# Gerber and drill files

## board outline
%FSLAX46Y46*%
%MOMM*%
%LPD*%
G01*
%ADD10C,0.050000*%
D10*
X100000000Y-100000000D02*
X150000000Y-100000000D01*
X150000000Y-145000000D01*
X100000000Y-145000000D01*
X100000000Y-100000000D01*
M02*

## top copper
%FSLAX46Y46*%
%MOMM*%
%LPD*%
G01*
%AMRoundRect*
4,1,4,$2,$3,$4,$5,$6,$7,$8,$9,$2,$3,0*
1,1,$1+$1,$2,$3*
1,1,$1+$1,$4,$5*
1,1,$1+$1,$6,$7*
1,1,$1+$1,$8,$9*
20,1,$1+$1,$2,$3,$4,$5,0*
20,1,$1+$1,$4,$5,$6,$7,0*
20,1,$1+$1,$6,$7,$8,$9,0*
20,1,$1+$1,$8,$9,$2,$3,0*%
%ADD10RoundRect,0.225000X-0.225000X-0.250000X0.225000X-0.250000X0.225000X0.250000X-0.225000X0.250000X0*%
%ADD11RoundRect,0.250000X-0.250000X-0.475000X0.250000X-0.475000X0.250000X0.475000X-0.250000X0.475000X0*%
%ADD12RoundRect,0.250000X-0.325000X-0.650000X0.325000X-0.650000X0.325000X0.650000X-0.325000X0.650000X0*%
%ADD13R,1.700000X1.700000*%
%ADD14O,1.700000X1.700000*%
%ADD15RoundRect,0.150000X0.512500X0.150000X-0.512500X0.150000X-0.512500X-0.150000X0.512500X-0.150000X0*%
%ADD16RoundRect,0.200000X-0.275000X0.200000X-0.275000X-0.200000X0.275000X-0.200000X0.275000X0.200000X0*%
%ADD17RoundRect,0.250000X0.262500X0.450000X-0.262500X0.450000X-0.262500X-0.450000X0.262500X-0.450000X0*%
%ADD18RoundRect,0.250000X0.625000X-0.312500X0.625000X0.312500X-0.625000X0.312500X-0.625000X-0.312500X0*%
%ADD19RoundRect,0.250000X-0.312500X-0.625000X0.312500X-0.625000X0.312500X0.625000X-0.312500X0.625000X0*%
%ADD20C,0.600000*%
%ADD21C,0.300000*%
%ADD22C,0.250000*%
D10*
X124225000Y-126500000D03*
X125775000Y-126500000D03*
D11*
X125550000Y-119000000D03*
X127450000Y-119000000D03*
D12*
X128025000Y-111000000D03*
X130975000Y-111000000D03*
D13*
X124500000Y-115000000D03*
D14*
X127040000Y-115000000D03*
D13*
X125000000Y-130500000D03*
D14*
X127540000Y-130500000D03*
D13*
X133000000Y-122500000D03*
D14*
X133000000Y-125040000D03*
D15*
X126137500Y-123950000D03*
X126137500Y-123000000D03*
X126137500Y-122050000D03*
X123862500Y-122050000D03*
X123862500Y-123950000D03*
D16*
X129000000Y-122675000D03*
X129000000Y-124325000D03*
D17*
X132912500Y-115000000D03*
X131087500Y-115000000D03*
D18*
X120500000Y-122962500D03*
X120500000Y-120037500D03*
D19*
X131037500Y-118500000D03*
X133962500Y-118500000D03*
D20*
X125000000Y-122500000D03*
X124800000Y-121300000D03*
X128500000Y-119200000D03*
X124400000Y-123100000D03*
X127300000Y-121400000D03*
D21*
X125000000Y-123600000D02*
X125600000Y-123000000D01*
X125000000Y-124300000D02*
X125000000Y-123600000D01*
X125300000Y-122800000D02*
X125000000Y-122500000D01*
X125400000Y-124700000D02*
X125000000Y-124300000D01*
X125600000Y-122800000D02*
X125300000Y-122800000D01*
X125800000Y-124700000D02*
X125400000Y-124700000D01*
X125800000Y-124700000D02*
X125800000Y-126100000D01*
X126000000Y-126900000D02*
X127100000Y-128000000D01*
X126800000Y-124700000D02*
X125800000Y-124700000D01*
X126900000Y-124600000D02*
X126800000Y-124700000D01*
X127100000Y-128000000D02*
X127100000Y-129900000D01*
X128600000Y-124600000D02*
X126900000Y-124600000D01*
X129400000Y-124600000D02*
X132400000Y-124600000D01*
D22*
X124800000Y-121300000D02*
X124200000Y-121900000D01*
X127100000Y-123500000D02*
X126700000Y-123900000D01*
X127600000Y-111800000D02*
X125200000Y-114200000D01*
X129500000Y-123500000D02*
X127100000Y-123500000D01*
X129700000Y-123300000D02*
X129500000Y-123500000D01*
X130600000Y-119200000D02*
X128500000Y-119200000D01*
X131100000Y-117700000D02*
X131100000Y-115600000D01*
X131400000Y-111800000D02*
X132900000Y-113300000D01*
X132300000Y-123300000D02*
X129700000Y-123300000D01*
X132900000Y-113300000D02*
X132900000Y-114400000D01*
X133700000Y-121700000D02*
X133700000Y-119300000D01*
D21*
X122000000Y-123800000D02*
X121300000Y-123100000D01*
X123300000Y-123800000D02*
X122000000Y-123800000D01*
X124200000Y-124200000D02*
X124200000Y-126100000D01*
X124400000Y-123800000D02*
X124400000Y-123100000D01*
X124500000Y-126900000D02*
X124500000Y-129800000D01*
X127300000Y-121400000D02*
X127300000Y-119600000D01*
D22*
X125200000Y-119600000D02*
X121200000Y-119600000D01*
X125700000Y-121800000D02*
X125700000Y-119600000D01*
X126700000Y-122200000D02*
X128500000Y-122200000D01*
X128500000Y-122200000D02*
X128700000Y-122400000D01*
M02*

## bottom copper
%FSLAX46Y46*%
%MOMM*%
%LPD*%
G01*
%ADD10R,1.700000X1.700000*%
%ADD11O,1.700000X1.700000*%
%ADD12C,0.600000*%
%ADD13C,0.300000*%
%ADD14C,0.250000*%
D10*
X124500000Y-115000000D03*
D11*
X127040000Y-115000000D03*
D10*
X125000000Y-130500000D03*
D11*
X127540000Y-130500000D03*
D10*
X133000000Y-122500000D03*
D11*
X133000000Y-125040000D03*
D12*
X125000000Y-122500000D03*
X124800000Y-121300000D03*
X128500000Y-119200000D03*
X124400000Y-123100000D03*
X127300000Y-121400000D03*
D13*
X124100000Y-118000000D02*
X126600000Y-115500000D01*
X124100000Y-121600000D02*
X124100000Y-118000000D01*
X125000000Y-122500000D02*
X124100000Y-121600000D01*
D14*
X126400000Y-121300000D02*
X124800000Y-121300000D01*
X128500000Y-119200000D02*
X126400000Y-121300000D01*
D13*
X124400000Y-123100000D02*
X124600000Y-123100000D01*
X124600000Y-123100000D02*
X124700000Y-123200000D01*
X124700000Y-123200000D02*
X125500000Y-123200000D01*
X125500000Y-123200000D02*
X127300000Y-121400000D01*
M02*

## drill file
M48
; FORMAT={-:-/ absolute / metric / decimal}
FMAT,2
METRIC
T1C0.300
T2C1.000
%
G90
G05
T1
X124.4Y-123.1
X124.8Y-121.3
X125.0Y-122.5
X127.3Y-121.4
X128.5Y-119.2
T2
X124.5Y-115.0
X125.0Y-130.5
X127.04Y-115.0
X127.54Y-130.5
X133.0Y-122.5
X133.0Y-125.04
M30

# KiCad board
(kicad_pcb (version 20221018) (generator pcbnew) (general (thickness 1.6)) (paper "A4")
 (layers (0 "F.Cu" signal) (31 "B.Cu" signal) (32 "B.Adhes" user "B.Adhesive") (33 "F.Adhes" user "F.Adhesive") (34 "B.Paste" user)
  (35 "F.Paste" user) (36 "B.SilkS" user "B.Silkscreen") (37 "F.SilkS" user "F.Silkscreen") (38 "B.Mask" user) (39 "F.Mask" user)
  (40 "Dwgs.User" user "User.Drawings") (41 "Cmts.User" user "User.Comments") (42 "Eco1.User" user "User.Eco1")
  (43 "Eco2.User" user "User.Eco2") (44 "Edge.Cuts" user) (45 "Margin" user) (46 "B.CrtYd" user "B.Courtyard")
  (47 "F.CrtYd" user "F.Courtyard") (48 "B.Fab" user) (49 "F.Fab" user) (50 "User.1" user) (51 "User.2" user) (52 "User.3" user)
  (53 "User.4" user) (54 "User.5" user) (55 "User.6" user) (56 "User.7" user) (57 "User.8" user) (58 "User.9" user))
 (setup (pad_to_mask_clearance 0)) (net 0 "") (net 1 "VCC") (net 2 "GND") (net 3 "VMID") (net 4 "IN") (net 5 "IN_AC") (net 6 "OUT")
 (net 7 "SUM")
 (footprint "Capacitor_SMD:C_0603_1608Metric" (layer "F.Cu") (at 125 126.5)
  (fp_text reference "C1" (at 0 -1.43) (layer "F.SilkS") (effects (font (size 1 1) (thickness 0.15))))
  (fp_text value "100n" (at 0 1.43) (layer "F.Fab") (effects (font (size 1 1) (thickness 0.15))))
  (pad "1" smd roundrect (at -0.775 0) (size 0.9 0.95) (layers "F.Cu" "F.Paste" "F.Mask") (roundrect_rratio 0.25) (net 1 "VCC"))
  (pad "2" smd roundrect (at 0.775 0) (size 0.9 0.95) (layers "F.Cu" "F.Paste" "F.Mask") (roundrect_rratio 0.25) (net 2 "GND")))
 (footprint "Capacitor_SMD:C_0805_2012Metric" (layer "F.Cu") (at 126.5 119)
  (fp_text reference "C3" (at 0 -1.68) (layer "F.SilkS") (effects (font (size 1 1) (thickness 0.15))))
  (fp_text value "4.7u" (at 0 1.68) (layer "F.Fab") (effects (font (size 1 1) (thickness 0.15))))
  (pad "1" smd roundrect (at -0.95 0) (size 1 1.45) (layers "F.Cu" "F.Paste" "F.Mask") (roundrect_rratio 0.25) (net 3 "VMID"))
  (pad "2" smd roundrect (at 0.95 0) (size 1 1.45) (layers "F.Cu" "F.Paste" "F.Mask") (roundrect_rratio 0.25) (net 1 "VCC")))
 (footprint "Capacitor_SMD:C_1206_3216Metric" (layer "F.Cu") (at 129.5 111)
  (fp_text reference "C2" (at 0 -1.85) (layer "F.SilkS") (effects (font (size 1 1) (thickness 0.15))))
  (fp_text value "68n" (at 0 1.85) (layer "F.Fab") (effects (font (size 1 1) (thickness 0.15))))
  (pad "1" smd roundrect (at -1.475 0) (size 1.15 1.8) (layers "F.Cu" "F.Paste" "F.Mask") (roundrect_rratio 0.217391) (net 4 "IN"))
  (pad "2" smd roundrect (at 1.475 0) (size 1.15 1.8) (layers "F.Cu" "F.Paste" "F.Mask") (roundrect_rratio 0.217391) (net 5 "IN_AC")))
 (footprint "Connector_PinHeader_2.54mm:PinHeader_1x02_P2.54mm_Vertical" (layer "F.Cu") (at 124.5 115 90)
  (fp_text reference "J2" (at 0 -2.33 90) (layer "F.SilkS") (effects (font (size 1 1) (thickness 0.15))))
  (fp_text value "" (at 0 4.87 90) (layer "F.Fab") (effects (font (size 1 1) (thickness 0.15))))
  (pad "1" thru_hole rect (at 0 0 90) (size 1.7 1.7) (drill 1) (layers "*.Cu" "*.Mask") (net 4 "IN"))
  (pad "2" thru_hole oval (at 0 2.54 90) (size 1.7 1.7) (drill 1) (layers "*.Cu" "*.Mask") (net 2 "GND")))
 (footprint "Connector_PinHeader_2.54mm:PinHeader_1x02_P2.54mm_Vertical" (layer "F.Cu") (at 125 130.5 90)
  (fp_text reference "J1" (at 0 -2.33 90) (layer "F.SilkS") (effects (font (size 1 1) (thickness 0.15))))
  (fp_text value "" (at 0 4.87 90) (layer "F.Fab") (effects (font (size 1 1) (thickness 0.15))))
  (pad "1" thru_hole rect (at 0 0 90) (size 1.7 1.7) (drill 1) (layers "*.Cu" "*.Mask") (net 1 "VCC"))
  (pad "2" thru_hole oval (at 0 2.54 90) (size 1.7 1.7) (drill 1) (layers "*.Cu" "*.Mask") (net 2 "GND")))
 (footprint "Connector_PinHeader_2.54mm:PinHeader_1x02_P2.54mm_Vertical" (layer "F.Cu") (at 133 122.5)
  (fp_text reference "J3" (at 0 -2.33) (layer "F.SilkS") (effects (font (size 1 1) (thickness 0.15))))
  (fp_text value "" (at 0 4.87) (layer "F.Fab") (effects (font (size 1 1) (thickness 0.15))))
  (pad "1" thru_hole rect (at 0 0) (size 1.7 1.7) (drill 1) (layers "*.Cu" "*.Mask") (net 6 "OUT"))
  (pad "2" thru_hole oval (at 0 2.54) (size 1.7 1.7) (drill 1) (layers "*.Cu" "*.Mask") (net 2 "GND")))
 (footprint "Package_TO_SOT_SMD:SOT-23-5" (layer "F.Cu") (at 125 123 180)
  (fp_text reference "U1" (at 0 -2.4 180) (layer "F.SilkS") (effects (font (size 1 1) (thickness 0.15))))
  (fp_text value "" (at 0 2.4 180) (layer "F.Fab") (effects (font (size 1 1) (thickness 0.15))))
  (pad "1" smd roundrect (at -1.1375 -0.95 180) (size 1.325 0.6) (layers "F.Cu" "F.Paste" "F.Mask") (roundrect_rratio 0.25) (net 6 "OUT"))
  (pad "2" smd roundrect (at -1.1375 0 180) (size 1.325 0.6) (layers "F.Cu" "F.Paste" "F.Mask") (roundrect_rratio 0.25) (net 2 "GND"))
  (pad "3" smd roundrect (at -1.1375 0.95 180) (size 1.325 0.6) (layers "F.Cu" "F.Paste" "F.Mask") (roundrect_rratio 0.25) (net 3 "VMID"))
  (pad "4" smd roundrect (at 1.1375 0.95 180) (size 1.325 0.6) (layers "F.Cu" "F.Paste" "F.Mask") (roundrect_rratio 0.25) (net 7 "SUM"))
  (pad "5" smd roundrect (at 1.1375 -0.95 180) (size 1.325 0.6) (layers "F.Cu" "F.Paste" "F.Mask") (roundrect_rratio 0.25) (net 1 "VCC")))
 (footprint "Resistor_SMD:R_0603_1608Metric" (layer "F.Cu") (at 129 123.5 -90)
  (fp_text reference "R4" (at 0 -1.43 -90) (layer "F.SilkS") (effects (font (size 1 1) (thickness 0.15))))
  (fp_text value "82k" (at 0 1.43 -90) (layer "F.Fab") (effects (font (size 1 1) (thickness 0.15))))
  (pad "1" smd roundrect (at -0.825 0 270) (size 0.8 0.95) (layers "F.Cu" "F.Paste" "F.Mask") (roundrect_rratio 0.25) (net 3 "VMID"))
  (pad "2" smd roundrect (at 0.825 0 270) (size 0.8 0.95) (layers "F.Cu" "F.Paste" "F.Mask") (roundrect_rratio 0.25) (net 2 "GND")))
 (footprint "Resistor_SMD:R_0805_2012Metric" (layer "F.Cu") (at 132 115 180)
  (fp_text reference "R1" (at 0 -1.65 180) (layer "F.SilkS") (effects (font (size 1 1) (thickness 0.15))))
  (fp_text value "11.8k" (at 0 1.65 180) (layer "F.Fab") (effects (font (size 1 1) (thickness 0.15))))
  (pad "1" smd roundrect (at -0.9125 0 180) (size 1.025 1.4) (layers "F.Cu" "F.Paste" "F.Mask") (roundrect_rratio 0.243902) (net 5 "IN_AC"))
  (pad "2" smd roundrect (at 0.9125 0 180) (size 1.025 1.4) (layers "F.Cu" "F.Paste" "F.Mask") (roundrect_rratio 0.243902) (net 7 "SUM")))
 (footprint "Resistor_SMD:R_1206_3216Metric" (layer "F.Cu") (at 120.5 121.5 90)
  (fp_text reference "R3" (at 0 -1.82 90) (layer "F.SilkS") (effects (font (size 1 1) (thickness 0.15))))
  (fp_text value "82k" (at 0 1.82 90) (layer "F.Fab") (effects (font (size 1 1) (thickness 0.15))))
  (pad "1" smd roundrect (at -1.4625 0 90) (size 1.125 1.75) (layers "F.Cu" "F.Paste" "F.Mask") (roundrect_rratio 0.222222) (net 1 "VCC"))
  (pad "2" smd roundrect (at 1.4625 0 90) (size 1.125 1.75) (layers "F.Cu" "F.Paste" "F.Mask") (roundrect_rratio 0.222222) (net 3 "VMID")))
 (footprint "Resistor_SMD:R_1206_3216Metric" (layer "F.Cu") (at 132.5 118.5)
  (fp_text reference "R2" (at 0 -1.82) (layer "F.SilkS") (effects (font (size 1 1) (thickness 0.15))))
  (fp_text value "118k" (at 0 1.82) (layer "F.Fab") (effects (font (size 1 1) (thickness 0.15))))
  (pad "1" smd roundrect (at -1.4625 0) (size 1.125 1.75) (layers "F.Cu" "F.Paste" "F.Mask") (roundrect_rratio 0.222222) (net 7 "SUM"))
  (pad "2" smd roundrect (at 1.4625 0) (size 1.125 1.75) (layers "F.Cu" "F.Paste" "F.Mask") (roundrect_rratio 0.222222) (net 6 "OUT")))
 (gr_rect (start 100 100) (end 150 145) (stroke (width 0.05) (type default)) (fill none) (layer "Edge.Cuts"))
 (segment (start 125 123.6) (end 125.6 123) (width 0.3) (layer "F.Cu") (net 2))
 (segment (start 125 124.3) (end 125 123.6) (width 0.3) (layer "F.Cu") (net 2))
 (segment (start 125.3 122.8) (end 125 122.5) (width 0.3) (layer "F.Cu") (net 2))
 (segment (start 125.4 124.7) (end 125 124.3) (width 0.3) (layer "F.Cu") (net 2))
 (segment (start 125.6 122.8) (end 125.3 122.8) (width 0.3) (layer "F.Cu") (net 2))
 (segment (start 125.8 124.7) (end 125.4 124.7) (width 0.3) (layer "F.Cu") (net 2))
 (segment (start 125.8 124.7) (end 125.8 126.1) (width 0.3) (layer "F.Cu") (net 2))
 (segment (start 126 126.9) (end 127.1 128) (width 0.3) (layer "F.Cu") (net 2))
 (segment (start 126.8 124.7) (end 125.8 124.7) (width 0.3) (layer "F.Cu") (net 2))
 (segment (start 126.9 124.6) (end 126.8 124.7) (width 0.3) (layer "F.Cu") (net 2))
 (segment (start 127.1 128) (end 127.1 129.9) (width 0.3) (layer "F.Cu") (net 2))
 (segment (start 128.6 124.6) (end 126.9 124.6) (width 0.3) (layer "F.Cu") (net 2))
 (segment (start 129.4 124.6) (end 132.4 124.6) (width 0.3) (layer "F.Cu") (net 2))
 (via (at 125 122.5) (size 0.6) (drill 0.3) (layers "F.Cu" "B.Cu") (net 2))
 (segment (start 124.1 118) (end 126.6 115.5) (width 0.3) (layer "B.Cu") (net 2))
 (segment (start 124.1 121.6) (end 124.1 118) (width 0.3) (layer "B.Cu") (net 2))
 (segment (start 124.8 121.3) (end 124.2 121.9) (width 0.25) (layer "F.Cu") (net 7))
 (segment (start 125 122.5) (end 124.1 121.6) (width 0.3) (layer "B.Cu") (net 2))
 (segment (start 127.1 123.5) (end 126.7 123.9) (width 0.25) (layer "F.Cu") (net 6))
 (segment (start 127.6 111.8) (end 125.2 114.2) (width 0.25) (layer "F.Cu") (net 4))
 (segment (start 129.5 123.5) (end 127.1 123.5) (width 0.25) (layer "F.Cu") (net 6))
 (segment (start 129.7 123.3) (end 129.5 123.5) (width 0.25) (layer "F.Cu") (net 6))
 (segment (start 130.6 119.2) (end 128.5 119.2) (width 0.25) (layer "F.Cu") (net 7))
 (segment (start 131.1 117.7) (end 131.1 115.6) (width 0.25) (layer "F.Cu") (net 7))
 (segment (start 131.4 111.8) (end 132.9 113.3) (width 0.25) (layer "F.Cu") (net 5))
 (segment (start 132.3 123.3) (end 129.7 123.3) (width 0.25) (layer "F.Cu") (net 6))
 (segment (start 132.9 113.3) (end 132.9 114.4) (width 0.25) (layer "F.Cu") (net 5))
 (segment (start 133.7 121.7) (end 133.7 119.3) (width 0.25) (layer "F.Cu") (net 6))
 (via (at 124.8 121.3) (size 0.6) (drill 0.3) (layers "F.Cu" "B.Cu") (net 7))
 (via (at 128.5 119.2) (size 0.6) (drill 0.3) (layers "F.Cu" "B.Cu") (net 7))
 (segment (start 122 123.8) (end 121.3 123.1) (width 0.3) (layer "F.Cu") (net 1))
 (segment (start 123.3 123.8) (end 122 123.8) (width 0.3) (layer "F.Cu") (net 1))
 (segment (start 124.2 124.2) (end 124.2 126.1) (width 0.3) (layer "F.Cu") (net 1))
 (segment (start 124.4 123.8) (end 124.4 123.1) (width 0.3) (layer "F.Cu") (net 1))
 (segment (start 124.5 126.9) (end 124.5 129.8) (width 0.3) (layer "F.Cu") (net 1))
 (segment (start 126.4 121.3) (end 124.8 121.3) (width 0.25) (layer "B.Cu") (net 7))
 (segment (start 127.3 121.4) (end 127.3 119.6) (width 0.3) (layer "F.Cu") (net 1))
 (segment (start 128.5 119.2) (end 126.4 121.3) (width 0.25) (layer "B.Cu") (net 7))
 (via (at 124.4 123.1) (size 0.6) (drill 0.3) (layers "F.Cu" "B.Cu") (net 1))
 (via (at 127.3 121.4) (size 0.6) (drill 0.3) (layers "F.Cu" "B.Cu") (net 1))
 (segment (start 124.4 123.1) (end 124.6 123.1) (width 0.3) (layer "B.Cu") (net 1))
 (segment (start 124.6 123.1) (end 124.7 123.2) (width 0.3) (layer "B.Cu") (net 1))
 (segment (start 124.7 123.2) (end 125.5 123.2) (width 0.3) (layer "B.Cu") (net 1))
 (segment (start 125.2 119.6) (end 121.2 119.6) (width 0.25) (layer "F.Cu") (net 3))
 (segment (start 125.5 123.2) (end 127.3 121.4) (width 0.3) (layer "B.Cu") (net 1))
 (segment (start 125.7 121.8) (end 125.7 119.6) (width 0.25) (layer "F.Cu") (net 3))
 (segment (start 126.7 122.2) (end 128.5 122.2) (width 0.25) (layer "F.Cu") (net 3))
 (segment (start 128.5 122.2) (end 128.7 122.4) (width 0.25) (layer "F.Cu") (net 3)))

